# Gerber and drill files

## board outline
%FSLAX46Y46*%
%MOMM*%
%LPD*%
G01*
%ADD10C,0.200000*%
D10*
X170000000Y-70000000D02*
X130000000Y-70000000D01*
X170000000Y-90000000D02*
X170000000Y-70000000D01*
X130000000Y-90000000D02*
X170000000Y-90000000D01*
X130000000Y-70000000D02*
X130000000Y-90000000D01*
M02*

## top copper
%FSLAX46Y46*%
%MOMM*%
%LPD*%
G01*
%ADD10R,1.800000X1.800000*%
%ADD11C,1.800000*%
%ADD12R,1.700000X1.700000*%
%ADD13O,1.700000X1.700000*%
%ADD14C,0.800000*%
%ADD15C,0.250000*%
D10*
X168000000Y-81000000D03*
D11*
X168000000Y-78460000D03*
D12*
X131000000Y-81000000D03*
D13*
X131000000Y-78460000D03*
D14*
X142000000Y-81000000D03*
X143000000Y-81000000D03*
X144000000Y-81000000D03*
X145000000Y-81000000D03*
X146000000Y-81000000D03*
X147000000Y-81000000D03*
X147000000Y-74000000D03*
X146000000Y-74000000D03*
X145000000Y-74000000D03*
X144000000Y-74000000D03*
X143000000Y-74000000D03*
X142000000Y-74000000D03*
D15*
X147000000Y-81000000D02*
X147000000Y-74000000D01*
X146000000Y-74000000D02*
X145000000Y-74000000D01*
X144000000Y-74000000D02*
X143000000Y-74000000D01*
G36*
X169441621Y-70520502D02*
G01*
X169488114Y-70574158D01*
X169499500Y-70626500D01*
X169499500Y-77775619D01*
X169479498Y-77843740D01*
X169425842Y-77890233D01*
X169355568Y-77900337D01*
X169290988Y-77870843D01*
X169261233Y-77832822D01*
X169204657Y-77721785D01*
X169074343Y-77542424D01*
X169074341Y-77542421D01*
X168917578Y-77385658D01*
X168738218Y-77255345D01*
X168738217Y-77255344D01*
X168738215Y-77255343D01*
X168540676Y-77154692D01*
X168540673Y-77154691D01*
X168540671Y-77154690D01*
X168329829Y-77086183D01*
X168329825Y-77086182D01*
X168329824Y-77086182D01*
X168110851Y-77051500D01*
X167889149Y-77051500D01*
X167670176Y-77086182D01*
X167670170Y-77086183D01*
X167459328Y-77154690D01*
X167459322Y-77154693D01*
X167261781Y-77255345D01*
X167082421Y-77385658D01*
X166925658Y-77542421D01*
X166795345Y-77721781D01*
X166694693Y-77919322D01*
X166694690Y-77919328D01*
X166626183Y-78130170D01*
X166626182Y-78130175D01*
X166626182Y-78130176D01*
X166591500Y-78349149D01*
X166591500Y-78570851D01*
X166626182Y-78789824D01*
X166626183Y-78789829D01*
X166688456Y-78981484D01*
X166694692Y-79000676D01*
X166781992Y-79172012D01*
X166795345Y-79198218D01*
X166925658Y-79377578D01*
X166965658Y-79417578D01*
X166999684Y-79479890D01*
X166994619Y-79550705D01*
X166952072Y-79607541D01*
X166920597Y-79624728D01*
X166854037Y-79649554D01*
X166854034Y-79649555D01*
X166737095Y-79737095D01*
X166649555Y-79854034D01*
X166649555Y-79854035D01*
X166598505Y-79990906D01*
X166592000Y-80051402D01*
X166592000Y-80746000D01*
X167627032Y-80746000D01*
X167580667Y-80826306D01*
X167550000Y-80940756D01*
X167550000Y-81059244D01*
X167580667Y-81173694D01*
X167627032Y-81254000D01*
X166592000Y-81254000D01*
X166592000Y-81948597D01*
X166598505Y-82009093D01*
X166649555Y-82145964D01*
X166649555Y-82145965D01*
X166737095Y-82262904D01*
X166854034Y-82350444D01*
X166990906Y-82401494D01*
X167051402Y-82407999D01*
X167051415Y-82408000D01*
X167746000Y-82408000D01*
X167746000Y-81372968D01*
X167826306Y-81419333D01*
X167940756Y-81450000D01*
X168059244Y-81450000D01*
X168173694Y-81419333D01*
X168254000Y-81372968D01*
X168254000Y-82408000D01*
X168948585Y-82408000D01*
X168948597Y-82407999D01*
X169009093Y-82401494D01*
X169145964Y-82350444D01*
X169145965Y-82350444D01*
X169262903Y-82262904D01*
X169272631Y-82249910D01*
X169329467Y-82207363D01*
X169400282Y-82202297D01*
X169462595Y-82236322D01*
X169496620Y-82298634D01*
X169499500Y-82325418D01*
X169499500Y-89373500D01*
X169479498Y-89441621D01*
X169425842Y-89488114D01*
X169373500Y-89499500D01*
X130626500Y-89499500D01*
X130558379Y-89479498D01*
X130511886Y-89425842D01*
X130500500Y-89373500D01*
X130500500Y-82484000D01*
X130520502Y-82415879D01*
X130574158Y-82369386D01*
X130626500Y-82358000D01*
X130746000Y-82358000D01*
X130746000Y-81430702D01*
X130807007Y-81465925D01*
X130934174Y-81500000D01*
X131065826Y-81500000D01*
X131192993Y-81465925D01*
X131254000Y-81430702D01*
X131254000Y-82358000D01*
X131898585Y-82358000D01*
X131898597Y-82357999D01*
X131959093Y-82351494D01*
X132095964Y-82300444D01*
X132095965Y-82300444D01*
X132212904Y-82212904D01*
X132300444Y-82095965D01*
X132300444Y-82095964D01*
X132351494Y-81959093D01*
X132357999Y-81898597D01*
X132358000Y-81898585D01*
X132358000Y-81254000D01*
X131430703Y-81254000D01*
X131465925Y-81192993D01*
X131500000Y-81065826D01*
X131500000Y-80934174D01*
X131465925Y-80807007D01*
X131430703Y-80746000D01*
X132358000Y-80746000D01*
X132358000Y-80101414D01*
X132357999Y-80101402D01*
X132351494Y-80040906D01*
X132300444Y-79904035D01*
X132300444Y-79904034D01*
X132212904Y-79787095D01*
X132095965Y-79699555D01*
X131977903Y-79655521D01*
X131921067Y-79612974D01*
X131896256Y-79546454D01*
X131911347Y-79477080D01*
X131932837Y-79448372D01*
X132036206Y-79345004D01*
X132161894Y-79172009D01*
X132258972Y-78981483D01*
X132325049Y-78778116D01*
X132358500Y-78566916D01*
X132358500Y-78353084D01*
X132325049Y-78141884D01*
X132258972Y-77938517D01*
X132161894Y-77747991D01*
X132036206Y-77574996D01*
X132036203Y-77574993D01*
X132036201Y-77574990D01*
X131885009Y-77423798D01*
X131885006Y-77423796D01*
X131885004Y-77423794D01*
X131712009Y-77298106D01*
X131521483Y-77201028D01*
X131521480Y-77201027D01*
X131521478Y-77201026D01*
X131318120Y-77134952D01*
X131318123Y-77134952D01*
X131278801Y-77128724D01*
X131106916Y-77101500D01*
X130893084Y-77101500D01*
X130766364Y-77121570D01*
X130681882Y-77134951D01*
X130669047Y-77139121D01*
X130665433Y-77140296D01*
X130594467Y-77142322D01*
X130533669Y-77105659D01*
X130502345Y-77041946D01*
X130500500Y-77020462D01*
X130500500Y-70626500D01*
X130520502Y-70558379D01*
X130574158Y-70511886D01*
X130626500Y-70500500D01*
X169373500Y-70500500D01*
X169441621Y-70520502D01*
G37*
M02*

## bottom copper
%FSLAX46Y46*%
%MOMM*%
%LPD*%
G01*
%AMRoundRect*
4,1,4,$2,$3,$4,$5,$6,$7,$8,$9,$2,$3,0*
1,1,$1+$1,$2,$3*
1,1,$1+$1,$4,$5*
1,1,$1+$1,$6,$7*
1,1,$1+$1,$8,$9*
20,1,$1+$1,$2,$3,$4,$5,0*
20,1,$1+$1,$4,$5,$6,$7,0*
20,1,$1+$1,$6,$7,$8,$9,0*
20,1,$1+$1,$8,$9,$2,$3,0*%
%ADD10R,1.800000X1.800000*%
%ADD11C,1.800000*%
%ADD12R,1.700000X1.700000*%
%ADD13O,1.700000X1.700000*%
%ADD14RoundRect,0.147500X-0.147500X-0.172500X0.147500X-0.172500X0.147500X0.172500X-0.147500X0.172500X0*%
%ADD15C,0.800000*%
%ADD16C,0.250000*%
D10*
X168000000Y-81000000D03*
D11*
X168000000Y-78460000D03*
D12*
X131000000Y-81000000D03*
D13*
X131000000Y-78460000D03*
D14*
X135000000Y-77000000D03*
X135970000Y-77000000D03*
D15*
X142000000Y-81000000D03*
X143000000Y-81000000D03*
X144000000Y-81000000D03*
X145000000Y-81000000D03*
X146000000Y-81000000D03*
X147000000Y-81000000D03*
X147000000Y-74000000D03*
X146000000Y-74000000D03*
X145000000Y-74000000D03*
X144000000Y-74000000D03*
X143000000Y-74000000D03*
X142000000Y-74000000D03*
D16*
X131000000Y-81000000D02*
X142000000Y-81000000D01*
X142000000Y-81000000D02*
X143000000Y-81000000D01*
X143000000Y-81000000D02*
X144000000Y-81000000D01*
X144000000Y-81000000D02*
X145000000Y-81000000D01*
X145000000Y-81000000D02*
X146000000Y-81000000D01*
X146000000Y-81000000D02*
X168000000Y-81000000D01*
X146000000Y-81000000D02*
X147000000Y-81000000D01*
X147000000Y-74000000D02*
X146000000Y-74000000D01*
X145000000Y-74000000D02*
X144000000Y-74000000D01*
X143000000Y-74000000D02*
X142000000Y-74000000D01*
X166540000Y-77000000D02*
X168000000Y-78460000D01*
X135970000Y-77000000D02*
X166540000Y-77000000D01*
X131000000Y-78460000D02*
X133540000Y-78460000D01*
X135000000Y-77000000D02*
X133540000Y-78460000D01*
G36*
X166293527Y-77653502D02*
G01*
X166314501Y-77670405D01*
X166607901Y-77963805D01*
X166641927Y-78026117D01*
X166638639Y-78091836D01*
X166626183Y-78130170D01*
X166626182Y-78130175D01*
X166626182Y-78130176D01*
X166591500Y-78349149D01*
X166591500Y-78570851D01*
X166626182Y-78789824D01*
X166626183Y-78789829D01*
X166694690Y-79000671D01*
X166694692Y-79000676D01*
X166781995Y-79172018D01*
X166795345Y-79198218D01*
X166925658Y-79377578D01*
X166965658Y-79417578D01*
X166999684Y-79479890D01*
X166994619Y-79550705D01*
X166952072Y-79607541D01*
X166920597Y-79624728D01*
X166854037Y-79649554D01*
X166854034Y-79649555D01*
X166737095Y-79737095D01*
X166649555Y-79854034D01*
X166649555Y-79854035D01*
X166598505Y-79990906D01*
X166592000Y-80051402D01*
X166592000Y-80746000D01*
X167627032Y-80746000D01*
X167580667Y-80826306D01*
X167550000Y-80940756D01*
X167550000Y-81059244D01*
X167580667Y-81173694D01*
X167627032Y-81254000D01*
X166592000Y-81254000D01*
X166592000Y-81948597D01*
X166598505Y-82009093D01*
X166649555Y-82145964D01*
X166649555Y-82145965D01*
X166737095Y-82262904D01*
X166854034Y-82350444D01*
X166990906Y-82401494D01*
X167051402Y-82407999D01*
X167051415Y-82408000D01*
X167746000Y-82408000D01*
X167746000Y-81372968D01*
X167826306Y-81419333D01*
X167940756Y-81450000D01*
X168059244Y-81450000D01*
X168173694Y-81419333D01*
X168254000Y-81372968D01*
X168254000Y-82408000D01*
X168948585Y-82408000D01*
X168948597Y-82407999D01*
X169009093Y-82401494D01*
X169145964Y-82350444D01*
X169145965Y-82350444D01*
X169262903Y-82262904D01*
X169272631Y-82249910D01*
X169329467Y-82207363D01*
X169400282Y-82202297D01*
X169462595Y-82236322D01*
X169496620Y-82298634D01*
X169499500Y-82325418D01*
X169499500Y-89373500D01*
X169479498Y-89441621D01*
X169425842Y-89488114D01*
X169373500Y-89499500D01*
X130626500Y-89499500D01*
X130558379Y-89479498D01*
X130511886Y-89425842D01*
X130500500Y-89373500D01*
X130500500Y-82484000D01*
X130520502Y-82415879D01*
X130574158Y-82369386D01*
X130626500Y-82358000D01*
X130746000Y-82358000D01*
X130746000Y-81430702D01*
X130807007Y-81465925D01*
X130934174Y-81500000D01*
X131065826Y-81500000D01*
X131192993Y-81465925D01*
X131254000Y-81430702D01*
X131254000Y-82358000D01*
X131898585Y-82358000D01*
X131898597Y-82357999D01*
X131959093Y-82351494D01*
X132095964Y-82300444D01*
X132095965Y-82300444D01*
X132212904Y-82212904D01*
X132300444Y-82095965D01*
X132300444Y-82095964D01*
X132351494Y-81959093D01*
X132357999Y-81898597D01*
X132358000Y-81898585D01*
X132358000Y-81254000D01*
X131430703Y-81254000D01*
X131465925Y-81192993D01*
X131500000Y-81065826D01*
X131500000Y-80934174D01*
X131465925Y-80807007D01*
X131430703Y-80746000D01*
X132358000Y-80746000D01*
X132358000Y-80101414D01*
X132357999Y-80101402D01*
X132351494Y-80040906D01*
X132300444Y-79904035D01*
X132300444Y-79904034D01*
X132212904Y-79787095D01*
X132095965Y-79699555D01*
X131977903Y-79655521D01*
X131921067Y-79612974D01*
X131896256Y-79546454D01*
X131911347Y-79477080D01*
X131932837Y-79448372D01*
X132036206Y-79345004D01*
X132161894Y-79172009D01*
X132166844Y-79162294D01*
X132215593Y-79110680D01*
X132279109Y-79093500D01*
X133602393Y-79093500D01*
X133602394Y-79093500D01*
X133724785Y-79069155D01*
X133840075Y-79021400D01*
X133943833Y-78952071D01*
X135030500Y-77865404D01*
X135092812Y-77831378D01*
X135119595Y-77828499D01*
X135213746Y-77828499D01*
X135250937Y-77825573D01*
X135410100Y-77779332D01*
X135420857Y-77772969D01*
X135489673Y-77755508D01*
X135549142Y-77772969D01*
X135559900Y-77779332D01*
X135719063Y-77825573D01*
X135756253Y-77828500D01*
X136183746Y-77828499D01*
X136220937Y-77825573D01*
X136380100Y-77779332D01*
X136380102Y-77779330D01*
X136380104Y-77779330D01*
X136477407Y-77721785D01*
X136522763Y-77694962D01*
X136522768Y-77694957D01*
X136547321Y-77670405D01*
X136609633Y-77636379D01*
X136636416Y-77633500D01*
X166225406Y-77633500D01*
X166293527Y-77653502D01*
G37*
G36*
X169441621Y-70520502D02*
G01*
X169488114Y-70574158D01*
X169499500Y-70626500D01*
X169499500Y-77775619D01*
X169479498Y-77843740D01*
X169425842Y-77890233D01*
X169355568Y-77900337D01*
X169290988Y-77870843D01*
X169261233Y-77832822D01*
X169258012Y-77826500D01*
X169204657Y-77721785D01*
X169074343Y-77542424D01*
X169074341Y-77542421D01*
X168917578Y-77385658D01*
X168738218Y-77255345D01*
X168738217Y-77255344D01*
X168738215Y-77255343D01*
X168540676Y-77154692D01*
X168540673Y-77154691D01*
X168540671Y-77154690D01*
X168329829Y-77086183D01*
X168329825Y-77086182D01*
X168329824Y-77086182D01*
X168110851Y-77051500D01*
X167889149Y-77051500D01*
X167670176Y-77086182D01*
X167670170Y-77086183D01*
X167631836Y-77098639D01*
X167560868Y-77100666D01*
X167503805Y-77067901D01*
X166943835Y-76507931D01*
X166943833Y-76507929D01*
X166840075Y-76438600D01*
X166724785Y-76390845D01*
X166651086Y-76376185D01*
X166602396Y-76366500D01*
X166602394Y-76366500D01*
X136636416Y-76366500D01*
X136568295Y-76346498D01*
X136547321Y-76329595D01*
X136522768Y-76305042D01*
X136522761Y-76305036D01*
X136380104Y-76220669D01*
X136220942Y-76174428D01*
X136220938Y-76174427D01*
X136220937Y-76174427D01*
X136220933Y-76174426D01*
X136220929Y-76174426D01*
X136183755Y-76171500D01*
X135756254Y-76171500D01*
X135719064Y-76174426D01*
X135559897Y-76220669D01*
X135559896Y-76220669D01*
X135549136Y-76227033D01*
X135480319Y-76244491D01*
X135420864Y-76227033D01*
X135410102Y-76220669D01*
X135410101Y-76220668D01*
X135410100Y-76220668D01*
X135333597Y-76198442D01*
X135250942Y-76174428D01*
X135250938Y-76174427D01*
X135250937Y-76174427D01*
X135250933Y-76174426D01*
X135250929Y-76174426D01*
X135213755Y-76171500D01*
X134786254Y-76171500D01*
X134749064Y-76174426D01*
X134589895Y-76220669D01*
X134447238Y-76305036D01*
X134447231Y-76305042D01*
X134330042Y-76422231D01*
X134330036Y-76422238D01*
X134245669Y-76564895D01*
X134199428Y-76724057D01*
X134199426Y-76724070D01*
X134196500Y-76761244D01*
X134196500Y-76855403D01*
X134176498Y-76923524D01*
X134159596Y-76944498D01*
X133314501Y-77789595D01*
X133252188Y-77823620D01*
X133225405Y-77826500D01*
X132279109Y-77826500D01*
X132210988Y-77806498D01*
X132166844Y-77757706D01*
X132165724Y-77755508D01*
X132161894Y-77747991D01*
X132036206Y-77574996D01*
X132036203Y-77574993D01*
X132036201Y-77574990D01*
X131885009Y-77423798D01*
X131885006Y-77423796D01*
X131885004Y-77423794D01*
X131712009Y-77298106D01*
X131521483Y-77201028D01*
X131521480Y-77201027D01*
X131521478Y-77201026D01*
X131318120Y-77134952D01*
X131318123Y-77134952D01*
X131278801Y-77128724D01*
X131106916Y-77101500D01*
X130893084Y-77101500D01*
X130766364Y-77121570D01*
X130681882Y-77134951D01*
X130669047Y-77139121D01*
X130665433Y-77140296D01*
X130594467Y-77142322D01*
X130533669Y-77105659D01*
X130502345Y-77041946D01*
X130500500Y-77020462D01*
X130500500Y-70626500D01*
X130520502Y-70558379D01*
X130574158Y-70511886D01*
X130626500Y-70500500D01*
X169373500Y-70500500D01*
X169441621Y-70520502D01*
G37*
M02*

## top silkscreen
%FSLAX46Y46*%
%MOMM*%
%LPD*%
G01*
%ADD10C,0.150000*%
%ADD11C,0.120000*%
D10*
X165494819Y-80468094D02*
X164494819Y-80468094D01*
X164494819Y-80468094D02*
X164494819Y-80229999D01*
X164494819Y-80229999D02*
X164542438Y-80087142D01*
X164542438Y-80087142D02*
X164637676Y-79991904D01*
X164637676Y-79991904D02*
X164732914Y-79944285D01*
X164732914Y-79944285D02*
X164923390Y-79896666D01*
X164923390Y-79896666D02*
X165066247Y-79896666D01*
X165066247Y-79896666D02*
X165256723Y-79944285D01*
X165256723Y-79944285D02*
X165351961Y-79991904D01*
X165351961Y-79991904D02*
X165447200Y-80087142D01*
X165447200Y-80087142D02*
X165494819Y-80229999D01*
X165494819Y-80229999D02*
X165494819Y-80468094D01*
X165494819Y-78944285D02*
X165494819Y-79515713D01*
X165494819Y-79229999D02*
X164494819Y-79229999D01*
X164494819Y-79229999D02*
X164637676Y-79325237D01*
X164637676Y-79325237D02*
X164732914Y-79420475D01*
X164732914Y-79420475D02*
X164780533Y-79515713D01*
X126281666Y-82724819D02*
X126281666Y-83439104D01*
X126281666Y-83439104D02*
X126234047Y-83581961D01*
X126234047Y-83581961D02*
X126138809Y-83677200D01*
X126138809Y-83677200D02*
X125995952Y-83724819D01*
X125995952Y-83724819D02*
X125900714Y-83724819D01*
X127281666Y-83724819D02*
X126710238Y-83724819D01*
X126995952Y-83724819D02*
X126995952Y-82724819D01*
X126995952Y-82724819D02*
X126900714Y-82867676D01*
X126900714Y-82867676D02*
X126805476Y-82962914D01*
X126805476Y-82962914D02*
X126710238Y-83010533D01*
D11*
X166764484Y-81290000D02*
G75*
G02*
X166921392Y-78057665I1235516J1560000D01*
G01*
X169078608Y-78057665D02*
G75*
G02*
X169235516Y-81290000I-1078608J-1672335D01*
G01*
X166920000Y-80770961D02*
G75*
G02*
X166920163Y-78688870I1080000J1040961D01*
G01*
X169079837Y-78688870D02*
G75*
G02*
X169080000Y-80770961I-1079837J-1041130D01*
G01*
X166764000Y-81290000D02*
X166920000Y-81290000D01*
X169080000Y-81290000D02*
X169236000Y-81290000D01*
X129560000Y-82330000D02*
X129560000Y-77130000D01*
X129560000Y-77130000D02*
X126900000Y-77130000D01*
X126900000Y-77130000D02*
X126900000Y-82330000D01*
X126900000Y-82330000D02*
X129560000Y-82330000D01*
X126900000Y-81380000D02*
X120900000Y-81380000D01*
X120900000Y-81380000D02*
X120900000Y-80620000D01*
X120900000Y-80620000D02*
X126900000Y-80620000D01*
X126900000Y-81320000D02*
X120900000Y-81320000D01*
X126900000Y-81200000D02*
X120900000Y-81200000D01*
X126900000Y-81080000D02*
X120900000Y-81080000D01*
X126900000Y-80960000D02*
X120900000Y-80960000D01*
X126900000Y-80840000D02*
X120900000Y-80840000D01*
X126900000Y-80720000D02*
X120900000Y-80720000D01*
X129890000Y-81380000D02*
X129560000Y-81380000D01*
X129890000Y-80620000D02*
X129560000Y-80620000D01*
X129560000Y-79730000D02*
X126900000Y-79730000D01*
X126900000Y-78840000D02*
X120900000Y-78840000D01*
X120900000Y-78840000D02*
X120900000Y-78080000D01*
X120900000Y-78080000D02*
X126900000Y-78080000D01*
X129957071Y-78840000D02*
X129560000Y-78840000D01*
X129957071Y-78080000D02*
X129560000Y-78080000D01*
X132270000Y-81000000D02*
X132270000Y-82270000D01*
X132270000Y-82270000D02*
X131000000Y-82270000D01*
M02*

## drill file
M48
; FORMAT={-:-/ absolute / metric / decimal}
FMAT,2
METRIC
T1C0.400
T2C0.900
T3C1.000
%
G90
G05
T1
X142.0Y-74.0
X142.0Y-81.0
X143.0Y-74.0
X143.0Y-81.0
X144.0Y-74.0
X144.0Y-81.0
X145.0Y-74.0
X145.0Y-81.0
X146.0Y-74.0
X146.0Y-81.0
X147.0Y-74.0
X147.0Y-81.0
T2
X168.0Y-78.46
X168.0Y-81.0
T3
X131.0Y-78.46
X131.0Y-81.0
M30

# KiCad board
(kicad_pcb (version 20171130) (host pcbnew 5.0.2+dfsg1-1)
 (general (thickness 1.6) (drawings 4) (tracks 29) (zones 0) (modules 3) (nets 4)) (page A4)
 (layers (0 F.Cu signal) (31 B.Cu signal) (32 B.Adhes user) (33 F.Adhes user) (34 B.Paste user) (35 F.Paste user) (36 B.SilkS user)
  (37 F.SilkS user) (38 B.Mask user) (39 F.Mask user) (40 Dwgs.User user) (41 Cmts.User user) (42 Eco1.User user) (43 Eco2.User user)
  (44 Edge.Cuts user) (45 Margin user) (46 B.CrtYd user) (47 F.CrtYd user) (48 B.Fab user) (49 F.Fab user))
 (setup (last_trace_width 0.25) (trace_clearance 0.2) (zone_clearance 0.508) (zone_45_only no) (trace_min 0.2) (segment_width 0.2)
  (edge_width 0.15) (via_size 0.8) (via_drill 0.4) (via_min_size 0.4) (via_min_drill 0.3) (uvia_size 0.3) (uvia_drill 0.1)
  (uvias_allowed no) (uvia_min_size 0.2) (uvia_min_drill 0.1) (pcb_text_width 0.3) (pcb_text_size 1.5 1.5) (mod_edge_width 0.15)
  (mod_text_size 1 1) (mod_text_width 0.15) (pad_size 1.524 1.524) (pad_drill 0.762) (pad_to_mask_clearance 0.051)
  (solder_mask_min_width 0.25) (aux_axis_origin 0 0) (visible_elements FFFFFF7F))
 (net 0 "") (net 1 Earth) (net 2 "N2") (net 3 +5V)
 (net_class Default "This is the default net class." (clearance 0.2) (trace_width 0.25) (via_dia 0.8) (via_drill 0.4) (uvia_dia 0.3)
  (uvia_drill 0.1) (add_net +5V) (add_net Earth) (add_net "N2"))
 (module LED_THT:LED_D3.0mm (layer F.Cu) (at 168 81 90)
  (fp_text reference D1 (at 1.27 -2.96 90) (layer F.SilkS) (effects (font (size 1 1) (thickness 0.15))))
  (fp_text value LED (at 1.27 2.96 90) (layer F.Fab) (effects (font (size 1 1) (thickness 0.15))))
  (fp_arc (start 1.27 0) (end -0.29 -1.235516) (angle 108.8) (layer F.SilkS) (width 0.12))
  (fp_arc (start 1.27 0) (end -0.29 1.235516) (angle -108.8) (layer F.SilkS) (width 0.12))
  (fp_arc (start 1.27 0) (end 0.229039 -1.08) (angle 87.9) (layer F.SilkS) (width 0.12))
  (fp_arc (start 1.27 0) (end 0.229039 1.08) (angle -87.9) (layer F.SilkS) (width 0.12))
  (fp_line (start -0.29 -1.236) (end -0.29 -1.08) (layer F.SilkS) (width 0.12))
  (fp_line (start -0.29 1.08) (end -0.29 1.236) (layer F.SilkS) (width 0.12))
  (pad 1 thru_hole rect (at 0 0 90) (size 1.8 1.8) (drill 0.9) (layers *.Cu *.Mask) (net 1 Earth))
  (pad 2 thru_hole circle (at 2.54 0 90) (size 1.8 1.8) (drill 0.9) (layers *.Cu *.Mask) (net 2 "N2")))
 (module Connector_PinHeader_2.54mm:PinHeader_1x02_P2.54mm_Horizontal (layer F.Cu) (at 131 81 180)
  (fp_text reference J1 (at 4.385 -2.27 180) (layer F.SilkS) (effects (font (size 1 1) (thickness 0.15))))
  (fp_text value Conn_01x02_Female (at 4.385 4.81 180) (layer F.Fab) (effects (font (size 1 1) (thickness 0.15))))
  (fp_line (start 1.44 -1.33) (end 1.44 3.87) (layer F.SilkS) (width 0.12))
  (fp_line (start 1.44 3.87) (end 4.1 3.87) (layer F.SilkS) (width 0.12))
  (fp_line (start 4.1 3.87) (end 4.1 -1.33) (layer F.SilkS) (width 0.12))
  (fp_line (start 4.1 -1.33) (end 1.44 -1.33) (layer F.SilkS) (width 0.12))
  (fp_line (start 4.1 -0.38) (end 10.1 -0.38) (layer F.SilkS) (width 0.12))
  (fp_line (start 10.1 -0.38) (end 10.1 0.38) (layer F.SilkS) (width 0.12))
  (fp_line (start 10.1 0.38) (end 4.1 0.38) (layer F.SilkS) (width 0.12))
  (fp_line (start 4.1 -0.32) (end 10.1 -0.32) (layer F.SilkS) (width 0.12))
  (fp_line (start 4.1 -0.2) (end 10.1 -0.2) (layer F.SilkS) (width 0.12))
  (fp_line (start 4.1 -0.08) (end 10.1 -0.08) (layer F.SilkS) (width 0.12))
  (fp_line (start 4.1 0.04) (end 10.1 0.04) (layer F.SilkS) (width 0.12))
  (fp_line (start 4.1 0.16) (end 10.1 0.16) (layer F.SilkS) (width 0.12))
  (fp_line (start 4.1 0.28) (end 10.1 0.28) (layer F.SilkS) (width 0.12))
  (fp_line (start 1.11 -0.38) (end 1.44 -0.38) (layer F.SilkS) (width 0.12))
  (fp_line (start 1.11 0.38) (end 1.44 0.38) (layer F.SilkS) (width 0.12))
  (fp_line (start 1.44 1.27) (end 4.1 1.27) (layer F.SilkS) (width 0.12))
  (fp_line (start 4.1 2.16) (end 10.1 2.16) (layer F.SilkS) (width 0.12))
  (fp_line (start 10.1 2.16) (end 10.1 2.92) (layer F.SilkS) (width 0.12))
  (fp_line (start 10.1 2.92) (end 4.1 2.92) (layer F.SilkS) (width 0.12))
  (fp_line (start 1.042929 2.16) (end 1.44 2.16) (layer F.SilkS) (width 0.12))
  (fp_line (start 1.042929 2.92) (end 1.44 2.92) (layer F.SilkS) (width 0.12))
  (fp_line (start -1.27 0) (end -1.27 -1.27) (layer F.SilkS) (width 0.12))
  (fp_line (start -1.27 -1.27) (end 0 -1.27) (layer F.SilkS) (width 0.12))
  (pad 1 thru_hole rect (at 0 0 180) (size 1.7 1.7) (drill 1) (layers *.Cu *.Mask) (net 1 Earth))
  (pad 2 thru_hole oval (at 0 2.54 180) (size 1.7 1.7) (drill 1) (layers *.Cu *.Mask) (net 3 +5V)))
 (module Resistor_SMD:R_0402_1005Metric (layer B.Cu) (at 135.485 77)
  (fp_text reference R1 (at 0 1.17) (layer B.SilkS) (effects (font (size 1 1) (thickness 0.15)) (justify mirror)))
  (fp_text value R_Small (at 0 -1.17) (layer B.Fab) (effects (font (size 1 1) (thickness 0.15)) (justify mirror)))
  (pad 1 smd roundrect (at -0.485 0) (size 0.59 0.64) (layers B.Cu B.Paste B.Mask) (roundrect_rratio 0.25) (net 3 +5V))
  (pad 2 smd roundrect (at 0.485 0) (size 0.59 0.64) (layers B.Cu B.Paste B.Mask) (roundrect_rratio 0.25) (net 2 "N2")))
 (gr_line (start 170 70) (end 130 70) (layer Edge.Cuts) (width 0.2))
 (gr_line (start 170 90) (end 170 70) (layer Edge.Cuts) (width 0.2))
 (gr_line (start 130 90) (end 170 90) (layer Edge.Cuts) (width 0.2))
 (gr_line (start 130 70) (end 130 90) (layer Edge.Cuts) (width 0.2))
 (via (at 142 81) (size 0.8) (drill 0.4) (layers F.Cu B.Cu) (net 1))
 (segment (start 131 81) (end 142 81) (width 0.25) (layer B.Cu) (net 1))
 (via (at 143 81) (size 0.8) (drill 0.4) (layers F.Cu B.Cu) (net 1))
 (segment (start 142 81) (end 143 81) (width 0.25) (layer B.Cu) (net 1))
 (via (at 144 81) (size 0.8) (drill 0.4) (layers F.Cu B.Cu) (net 1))
 (segment (start 143 81) (end 144 81) (width 0.25) (layer B.Cu) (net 1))
 (via (at 145 81) (size 0.8) (drill 0.4) (layers F.Cu B.Cu) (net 1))
 (segment (start 144 81) (end 145 81) (width 0.25) (layer B.Cu) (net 1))
 (via (at 146 81) (size 0.8) (drill 0.4) (layers F.Cu B.Cu) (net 1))
 (segment (start 145 81) (end 146 81) (width 0.25) (layer B.Cu) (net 1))
 (segment (start 146 81) (end 168 81) (width 0.25) (layer B.Cu) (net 1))
 (via (at 147 81) (size 0.8) (drill 0.4) (layers F.Cu B.Cu) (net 1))
 (segment (start 146 81) (end 147 81) (width 0.25) (layer B.Cu) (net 1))
 (via (at 147 74) (size 0.8) (drill 0.4) (layers F.Cu B.Cu) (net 1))
 (segment (start 147 81) (end 147 74) (width 0.25) (layer F.Cu) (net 1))
 (via (at 146 74) (size 0.8) (drill 0.4) (layers F.Cu B.Cu) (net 1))
 (segment (start 147 74) (end 146 74) (width 0.25) (layer B.Cu) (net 1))
 (via (at 145 74) (size 0.8) (drill 0.4) (layers F.Cu B.Cu) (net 1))
 (segment (start 146 74) (end 145 74) (width 0.25) (layer F.Cu) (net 1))
 (via (at 144 74) (size 0.8) (drill 0.4) (layers F.Cu B.Cu) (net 1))
 (segment (start 145 74) (end 144 74) (width 0.25) (layer B.Cu) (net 1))
 (via (at 143 74) (size 0.8) (drill 0.4) (layers F.Cu B.Cu) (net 1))
 (segment (start 144 74) (end 143 74) (width 0.25) (layer F.Cu) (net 1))
 (via (at 142 74) (size 0.8) (drill 0.4) (layers F.Cu B.Cu) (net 1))
 (segment (start 143 74) (end 142 74) (width 0.25) (layer B.Cu) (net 1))
 (segment (start 166.54 77) (end 168 78.46) (width 0.25) (layer B.Cu) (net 2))
 (segment (start 135.97 77) (end 166.54 77) (width 0.25) (layer B.Cu) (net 2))
 (segment (start 131 78.46) (end 133.54 78.46) (width 0.25) (layer B.Cu) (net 3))
 (segment (start 135 77) (end 133.54 78.46) (width 0.25) (layer B.Cu) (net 3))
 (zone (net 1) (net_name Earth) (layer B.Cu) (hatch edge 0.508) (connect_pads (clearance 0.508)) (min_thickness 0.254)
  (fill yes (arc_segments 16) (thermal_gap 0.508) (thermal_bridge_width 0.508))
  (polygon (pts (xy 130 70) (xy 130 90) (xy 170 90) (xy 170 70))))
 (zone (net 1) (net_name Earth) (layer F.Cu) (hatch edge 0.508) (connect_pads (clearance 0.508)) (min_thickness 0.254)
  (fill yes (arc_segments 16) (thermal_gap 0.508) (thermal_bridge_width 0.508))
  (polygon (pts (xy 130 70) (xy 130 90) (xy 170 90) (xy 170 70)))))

